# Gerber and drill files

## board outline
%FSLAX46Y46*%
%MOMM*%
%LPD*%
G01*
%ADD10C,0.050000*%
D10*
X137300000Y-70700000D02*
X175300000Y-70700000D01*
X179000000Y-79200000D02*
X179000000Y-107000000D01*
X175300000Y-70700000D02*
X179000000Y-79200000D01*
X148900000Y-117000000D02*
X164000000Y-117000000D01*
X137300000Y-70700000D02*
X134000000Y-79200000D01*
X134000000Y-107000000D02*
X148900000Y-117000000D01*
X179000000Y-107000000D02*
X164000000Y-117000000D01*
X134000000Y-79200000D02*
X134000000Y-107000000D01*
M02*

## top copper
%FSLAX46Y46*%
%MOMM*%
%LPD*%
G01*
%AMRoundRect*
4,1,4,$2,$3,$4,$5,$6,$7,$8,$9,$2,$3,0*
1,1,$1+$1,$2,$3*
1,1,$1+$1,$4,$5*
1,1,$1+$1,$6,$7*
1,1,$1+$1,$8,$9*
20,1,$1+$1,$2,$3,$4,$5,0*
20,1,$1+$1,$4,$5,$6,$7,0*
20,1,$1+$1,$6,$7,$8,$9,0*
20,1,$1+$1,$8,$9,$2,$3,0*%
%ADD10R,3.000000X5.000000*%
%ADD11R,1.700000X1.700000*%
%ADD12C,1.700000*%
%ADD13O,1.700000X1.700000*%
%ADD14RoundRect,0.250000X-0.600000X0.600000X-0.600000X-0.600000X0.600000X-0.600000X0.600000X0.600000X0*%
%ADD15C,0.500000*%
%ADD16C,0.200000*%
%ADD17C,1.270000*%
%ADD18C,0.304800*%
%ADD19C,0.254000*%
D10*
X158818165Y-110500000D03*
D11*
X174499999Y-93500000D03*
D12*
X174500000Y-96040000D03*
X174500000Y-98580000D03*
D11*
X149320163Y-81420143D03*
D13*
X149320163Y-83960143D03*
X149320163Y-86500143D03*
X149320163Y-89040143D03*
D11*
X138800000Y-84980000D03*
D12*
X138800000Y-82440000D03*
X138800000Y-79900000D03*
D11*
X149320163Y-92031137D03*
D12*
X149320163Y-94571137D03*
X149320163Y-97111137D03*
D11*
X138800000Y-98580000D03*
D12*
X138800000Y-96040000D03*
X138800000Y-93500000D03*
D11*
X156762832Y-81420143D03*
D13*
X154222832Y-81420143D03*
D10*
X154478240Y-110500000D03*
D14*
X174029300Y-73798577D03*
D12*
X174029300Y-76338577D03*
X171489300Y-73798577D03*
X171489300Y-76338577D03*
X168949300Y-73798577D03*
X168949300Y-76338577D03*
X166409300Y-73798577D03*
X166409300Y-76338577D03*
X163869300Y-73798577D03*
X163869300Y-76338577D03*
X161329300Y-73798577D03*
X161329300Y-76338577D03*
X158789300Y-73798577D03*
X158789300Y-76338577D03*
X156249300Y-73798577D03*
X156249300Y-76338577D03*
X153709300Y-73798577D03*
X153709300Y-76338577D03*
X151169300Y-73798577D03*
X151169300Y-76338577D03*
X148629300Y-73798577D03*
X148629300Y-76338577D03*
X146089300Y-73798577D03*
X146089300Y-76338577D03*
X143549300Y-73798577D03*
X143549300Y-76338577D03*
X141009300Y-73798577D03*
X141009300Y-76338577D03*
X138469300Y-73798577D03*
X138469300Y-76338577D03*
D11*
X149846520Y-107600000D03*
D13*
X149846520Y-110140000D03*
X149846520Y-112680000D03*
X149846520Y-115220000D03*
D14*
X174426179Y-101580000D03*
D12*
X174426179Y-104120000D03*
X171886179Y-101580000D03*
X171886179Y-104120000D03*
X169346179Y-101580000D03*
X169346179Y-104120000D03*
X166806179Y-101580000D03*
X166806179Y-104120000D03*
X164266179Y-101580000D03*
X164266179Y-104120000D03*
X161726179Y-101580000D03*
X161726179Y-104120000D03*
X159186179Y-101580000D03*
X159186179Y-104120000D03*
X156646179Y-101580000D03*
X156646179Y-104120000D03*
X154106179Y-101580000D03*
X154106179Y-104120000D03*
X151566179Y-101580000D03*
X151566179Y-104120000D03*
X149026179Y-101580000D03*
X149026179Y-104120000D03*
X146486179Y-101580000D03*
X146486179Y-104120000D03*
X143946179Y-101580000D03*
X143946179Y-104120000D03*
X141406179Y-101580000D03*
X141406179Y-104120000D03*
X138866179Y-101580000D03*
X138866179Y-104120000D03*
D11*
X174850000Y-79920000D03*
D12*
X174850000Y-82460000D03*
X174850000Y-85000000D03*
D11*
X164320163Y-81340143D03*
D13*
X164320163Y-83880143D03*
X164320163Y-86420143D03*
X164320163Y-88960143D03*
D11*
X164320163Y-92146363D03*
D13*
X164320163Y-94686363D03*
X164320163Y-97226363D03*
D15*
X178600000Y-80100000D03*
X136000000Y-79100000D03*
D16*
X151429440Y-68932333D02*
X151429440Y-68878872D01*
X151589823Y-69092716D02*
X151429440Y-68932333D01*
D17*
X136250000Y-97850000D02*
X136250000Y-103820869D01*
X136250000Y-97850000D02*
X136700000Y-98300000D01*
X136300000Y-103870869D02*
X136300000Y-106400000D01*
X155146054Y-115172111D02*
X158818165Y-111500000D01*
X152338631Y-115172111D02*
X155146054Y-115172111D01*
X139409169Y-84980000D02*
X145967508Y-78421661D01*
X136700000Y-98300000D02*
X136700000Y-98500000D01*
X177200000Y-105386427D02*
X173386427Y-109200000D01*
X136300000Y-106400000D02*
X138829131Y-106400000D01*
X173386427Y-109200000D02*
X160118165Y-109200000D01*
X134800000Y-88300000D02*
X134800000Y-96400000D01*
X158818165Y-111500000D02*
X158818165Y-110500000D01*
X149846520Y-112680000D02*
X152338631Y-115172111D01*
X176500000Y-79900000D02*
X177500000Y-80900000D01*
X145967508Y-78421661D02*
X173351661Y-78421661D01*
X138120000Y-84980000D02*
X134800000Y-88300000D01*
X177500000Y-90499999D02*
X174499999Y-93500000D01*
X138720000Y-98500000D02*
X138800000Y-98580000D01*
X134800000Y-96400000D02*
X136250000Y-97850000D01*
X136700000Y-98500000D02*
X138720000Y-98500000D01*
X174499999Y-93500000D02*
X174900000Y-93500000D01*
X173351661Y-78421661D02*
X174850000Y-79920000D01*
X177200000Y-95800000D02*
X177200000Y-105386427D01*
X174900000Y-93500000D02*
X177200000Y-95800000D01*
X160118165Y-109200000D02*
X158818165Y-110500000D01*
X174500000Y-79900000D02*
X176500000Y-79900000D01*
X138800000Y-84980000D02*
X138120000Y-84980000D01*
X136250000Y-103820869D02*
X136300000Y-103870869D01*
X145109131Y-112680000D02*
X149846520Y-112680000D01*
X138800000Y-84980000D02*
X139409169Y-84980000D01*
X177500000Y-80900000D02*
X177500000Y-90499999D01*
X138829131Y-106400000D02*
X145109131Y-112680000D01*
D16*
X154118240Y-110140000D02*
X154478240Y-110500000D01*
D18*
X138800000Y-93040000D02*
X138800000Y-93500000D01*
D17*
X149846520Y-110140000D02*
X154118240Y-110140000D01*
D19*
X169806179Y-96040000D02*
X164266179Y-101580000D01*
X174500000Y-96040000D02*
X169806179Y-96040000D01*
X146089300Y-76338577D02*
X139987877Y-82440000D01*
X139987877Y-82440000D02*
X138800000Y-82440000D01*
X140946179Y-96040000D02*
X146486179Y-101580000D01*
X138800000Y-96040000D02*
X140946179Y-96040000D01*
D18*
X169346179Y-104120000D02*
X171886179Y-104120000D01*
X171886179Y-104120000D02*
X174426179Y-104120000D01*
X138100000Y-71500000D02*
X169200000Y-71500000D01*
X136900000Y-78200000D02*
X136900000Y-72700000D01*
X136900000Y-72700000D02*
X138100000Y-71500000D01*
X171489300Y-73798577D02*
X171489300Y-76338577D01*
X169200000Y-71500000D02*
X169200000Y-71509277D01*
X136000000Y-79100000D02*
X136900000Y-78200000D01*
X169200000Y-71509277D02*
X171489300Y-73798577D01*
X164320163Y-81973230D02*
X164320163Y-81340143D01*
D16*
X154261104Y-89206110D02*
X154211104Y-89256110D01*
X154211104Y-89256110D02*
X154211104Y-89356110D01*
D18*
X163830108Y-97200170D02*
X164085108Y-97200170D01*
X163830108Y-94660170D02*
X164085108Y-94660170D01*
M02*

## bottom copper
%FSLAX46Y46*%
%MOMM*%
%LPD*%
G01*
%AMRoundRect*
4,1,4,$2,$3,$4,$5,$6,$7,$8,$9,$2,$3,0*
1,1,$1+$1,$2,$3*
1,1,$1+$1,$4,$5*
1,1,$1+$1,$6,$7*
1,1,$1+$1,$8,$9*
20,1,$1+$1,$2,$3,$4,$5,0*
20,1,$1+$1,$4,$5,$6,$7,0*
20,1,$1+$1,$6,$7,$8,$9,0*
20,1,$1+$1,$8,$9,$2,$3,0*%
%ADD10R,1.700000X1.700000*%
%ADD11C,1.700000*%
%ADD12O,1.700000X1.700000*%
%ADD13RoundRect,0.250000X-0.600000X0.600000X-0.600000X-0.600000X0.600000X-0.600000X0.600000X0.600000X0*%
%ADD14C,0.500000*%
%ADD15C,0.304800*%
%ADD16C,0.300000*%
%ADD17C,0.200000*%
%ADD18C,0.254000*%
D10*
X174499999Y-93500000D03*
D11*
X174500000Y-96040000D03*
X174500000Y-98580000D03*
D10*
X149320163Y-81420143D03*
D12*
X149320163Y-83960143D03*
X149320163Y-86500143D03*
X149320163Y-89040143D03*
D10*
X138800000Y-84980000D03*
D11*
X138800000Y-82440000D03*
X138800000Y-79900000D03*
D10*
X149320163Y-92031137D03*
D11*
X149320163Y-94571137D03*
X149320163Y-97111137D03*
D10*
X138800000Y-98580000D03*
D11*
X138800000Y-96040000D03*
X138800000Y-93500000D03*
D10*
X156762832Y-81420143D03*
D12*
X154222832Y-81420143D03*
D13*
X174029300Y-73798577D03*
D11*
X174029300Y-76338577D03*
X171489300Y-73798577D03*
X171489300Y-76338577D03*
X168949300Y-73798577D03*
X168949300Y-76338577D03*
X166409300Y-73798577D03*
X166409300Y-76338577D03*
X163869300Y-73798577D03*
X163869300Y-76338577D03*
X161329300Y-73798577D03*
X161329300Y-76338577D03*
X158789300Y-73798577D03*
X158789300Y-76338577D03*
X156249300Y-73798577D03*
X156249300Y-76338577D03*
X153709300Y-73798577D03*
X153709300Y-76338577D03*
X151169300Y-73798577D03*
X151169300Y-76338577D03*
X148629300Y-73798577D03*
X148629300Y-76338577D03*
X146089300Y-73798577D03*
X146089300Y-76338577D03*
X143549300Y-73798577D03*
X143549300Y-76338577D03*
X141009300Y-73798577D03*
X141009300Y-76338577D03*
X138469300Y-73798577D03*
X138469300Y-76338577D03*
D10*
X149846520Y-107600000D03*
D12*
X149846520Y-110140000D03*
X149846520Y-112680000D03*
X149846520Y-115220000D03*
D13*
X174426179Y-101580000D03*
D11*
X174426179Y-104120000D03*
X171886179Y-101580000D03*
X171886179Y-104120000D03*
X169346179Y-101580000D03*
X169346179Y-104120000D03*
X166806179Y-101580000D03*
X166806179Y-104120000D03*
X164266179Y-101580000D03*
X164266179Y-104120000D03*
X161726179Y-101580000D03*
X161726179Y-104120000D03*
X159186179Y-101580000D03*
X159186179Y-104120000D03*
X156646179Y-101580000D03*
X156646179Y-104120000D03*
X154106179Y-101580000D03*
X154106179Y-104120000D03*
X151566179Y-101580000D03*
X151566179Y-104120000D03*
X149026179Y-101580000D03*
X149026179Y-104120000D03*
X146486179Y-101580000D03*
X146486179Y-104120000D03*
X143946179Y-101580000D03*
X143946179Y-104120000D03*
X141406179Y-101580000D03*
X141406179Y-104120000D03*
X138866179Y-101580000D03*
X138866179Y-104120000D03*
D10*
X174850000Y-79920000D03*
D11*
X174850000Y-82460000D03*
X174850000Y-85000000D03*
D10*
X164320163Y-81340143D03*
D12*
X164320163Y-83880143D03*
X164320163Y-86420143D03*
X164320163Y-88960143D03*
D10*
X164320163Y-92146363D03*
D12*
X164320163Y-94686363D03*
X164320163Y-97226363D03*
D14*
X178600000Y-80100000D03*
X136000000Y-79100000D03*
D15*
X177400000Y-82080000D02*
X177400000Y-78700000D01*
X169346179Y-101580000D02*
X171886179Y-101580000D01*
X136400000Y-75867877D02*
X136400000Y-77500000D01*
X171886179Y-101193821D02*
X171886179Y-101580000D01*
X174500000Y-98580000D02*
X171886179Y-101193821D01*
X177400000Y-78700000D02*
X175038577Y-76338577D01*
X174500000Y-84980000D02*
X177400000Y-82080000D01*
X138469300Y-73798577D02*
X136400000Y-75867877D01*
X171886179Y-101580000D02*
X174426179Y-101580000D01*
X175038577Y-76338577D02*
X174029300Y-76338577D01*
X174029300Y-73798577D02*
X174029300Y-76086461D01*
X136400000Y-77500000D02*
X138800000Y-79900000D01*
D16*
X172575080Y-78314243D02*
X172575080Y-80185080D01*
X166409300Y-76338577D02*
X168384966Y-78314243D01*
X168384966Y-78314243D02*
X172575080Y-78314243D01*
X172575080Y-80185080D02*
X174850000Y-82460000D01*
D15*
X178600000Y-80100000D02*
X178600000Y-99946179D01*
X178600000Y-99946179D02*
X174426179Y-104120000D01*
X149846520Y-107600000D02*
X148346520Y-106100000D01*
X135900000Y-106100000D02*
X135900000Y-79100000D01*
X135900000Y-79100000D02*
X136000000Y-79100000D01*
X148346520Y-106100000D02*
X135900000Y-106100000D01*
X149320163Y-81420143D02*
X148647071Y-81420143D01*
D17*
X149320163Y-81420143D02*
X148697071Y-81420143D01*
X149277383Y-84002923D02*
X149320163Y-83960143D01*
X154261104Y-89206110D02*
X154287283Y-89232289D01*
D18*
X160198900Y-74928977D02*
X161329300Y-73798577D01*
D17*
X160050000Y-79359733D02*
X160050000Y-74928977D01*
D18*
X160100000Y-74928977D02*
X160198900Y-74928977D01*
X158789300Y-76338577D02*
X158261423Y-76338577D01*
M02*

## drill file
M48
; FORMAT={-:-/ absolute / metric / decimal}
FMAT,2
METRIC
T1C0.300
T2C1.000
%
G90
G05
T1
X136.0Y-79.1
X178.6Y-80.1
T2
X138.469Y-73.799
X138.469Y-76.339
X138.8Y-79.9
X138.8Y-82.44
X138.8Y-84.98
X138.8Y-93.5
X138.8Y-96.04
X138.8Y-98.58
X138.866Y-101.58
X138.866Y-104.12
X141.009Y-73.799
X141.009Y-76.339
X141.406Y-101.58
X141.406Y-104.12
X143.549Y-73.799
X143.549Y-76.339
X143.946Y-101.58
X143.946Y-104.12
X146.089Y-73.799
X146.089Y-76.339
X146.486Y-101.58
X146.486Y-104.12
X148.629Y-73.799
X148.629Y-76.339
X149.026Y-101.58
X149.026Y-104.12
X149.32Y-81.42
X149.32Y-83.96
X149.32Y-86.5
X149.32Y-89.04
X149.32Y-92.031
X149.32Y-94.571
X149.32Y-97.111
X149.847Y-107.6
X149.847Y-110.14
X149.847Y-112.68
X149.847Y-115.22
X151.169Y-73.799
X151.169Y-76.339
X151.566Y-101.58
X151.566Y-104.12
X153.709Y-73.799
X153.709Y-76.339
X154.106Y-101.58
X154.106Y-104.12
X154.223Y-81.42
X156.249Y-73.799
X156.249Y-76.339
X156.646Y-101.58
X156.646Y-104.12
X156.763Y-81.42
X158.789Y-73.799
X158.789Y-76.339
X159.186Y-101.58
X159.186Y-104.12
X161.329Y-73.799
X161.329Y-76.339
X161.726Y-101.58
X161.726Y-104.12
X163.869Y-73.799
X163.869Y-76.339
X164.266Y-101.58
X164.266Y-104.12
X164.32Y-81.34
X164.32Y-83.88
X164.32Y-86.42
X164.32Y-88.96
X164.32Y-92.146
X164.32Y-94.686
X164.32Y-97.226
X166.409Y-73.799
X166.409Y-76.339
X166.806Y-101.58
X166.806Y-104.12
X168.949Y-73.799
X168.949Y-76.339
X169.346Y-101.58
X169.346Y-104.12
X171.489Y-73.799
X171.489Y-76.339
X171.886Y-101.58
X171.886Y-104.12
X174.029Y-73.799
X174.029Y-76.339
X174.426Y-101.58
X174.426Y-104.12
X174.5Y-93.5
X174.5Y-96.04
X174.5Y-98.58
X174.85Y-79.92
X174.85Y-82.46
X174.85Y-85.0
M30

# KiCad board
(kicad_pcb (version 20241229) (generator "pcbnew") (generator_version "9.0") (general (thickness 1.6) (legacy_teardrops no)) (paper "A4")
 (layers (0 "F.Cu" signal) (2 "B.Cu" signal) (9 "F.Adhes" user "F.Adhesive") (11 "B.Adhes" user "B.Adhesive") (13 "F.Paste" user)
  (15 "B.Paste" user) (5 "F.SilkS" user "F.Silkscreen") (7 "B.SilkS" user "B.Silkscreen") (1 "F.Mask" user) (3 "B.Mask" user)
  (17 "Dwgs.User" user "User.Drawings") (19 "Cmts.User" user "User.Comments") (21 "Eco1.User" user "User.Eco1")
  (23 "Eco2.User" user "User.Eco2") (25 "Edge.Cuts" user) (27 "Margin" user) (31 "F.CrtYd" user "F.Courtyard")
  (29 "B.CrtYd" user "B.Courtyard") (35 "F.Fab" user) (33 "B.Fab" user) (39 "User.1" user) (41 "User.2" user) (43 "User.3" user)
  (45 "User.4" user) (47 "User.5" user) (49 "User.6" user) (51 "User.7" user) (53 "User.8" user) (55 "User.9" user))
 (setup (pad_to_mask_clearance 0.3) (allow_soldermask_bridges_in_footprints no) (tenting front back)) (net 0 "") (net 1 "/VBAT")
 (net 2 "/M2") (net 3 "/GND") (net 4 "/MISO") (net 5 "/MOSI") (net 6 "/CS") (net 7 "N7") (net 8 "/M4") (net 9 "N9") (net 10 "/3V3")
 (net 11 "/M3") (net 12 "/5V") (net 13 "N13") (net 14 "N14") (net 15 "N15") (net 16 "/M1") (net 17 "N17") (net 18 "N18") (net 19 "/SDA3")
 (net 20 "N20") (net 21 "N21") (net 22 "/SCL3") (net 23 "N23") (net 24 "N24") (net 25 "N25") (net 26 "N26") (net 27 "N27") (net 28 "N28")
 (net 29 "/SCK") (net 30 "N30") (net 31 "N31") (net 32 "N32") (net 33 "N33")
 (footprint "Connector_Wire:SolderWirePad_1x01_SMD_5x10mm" (layer "F.Cu") (at 158.918165 105.046585)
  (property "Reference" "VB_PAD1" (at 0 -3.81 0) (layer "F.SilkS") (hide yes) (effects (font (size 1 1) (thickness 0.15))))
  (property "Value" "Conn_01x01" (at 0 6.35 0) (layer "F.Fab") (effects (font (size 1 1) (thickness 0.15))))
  (pad "1" smd rect (at -0.1 5.453415) (size 3 5) (layers "F.Cu" "F.Mask" "F.Paste") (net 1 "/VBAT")))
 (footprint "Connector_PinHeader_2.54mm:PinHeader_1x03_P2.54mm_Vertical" (layer "F.Cu") (at 170.094208 95.970955 -45)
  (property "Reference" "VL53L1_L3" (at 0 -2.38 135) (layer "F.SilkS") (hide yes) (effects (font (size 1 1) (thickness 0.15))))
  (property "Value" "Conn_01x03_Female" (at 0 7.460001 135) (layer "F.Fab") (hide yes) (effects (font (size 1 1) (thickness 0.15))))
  (pad "1" thru_hole rect (at 1.368136 -4.862594) (size 1.7 1.7) (drill 1) (layers "*.Cu" "*.Mask") (remove_unused_layers no)
   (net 1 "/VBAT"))
  (pad "2" thru_hole circle (at 3.164188 -3.066543 315) (size 1.7 1.7) (drill 1) (layers "*.Cu" "*.Mask") (remove_unused_layers no)
   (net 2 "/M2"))
  (pad "3" thru_hole circle (at 4.960239 -1.270492 315) (size 1.7 1.7) (drill 1) (layers "*.Cu" "*.Mask") (remove_unused_layers no)
   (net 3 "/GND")))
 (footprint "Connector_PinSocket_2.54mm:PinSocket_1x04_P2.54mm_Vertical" (layer "F.Cu") (at 149.320163 81.420143)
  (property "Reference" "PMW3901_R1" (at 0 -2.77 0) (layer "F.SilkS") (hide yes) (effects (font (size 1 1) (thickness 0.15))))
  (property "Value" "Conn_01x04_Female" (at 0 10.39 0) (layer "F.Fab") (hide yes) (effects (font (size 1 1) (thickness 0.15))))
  (pad "1" thru_hole rect (at 0 0) (size 1.7 1.7) (drill 1) (layers "*.Cu" "*.Mask") (remove_unused_layers no) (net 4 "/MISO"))
  (pad "2" thru_hole oval (at 0 2.54) (size 1.7 1.7) (drill 1) (layers "*.Cu" "*.Mask") (remove_unused_layers no) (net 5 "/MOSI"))
  (pad "3" thru_hole oval (at 0 5.08) (size 1.7 1.7) (drill 1) (layers "*.Cu" "*.Mask") (remove_unused_layers no) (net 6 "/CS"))
  (pad "4" thru_hole oval (at 0 7.62) (size 1.7 1.7) (drill 1) (layers "*.Cu" "*.Mask") (remove_unused_layers no) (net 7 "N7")))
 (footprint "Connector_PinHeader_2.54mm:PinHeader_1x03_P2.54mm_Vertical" (layer "F.Cu") (at 138.5 84.8 -45)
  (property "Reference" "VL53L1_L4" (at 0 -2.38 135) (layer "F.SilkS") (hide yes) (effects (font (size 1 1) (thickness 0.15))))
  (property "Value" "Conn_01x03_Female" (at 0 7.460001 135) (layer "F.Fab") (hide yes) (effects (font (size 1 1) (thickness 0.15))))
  (pad "1" thru_hole rect (at 0.339411 -0.084853 270) (size 1.7 1.7) (drill 1) (layers "*.Cu" "*.Mask") (remove_unused_layers no)
   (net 1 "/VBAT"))
  (pad "2" thru_hole circle (at -1.45664 -1.880904 315) (size 1.7 1.7) (drill 1) (layers "*.Cu" "*.Mask") (remove_unused_layers no)
   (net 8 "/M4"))
  (pad "3" thru_hole circle (at -3.252691 -3.676955 315) (size 1.7 1.7) (drill 1) (layers "*.Cu" "*.Mask") (remove_unused_layers no)
   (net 3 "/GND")))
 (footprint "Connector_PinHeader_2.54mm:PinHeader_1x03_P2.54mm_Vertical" (layer "F.Cu") (at 149.320163 92.031137)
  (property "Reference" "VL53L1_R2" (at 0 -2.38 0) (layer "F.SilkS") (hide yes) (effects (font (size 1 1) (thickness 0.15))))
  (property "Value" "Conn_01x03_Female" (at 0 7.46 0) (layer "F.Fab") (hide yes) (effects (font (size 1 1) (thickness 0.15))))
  (pad "1" thru_hole rect (at 0 0) (size 1.7 1.7) (drill 1) (layers "*.Cu" "*.Mask") (remove_unused_layers no) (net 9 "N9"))
  (pad "2" thru_hole circle (at 0 2.54) (size 1.7 1.7) (drill 1) (layers "*.Cu" "*.Mask") (remove_unused_layers no) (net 3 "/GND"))
  (pad "3" thru_hole circle (at 0 5.08) (size 1.7 1.7) (drill 1) (layers "*.Cu" "*.Mask") (remove_unused_layers no) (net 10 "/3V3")))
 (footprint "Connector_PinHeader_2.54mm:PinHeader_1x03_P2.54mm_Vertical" (layer "F.Cu") (at 142.775639 98.946265 -135)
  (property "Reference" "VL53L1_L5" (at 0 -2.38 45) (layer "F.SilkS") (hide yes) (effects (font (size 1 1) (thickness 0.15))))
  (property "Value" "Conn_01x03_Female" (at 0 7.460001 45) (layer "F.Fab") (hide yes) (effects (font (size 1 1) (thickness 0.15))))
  (pad "1" thru_hole rect (at 2.552213 3.07019 270) (size 1.7 1.7) (drill 1) (layers "*.Cu" "*.Mask") (remove_unused_layers no)
   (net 1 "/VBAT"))
  (pad "2" thru_hole circle (at 0.756162 4.866241 225) (size 1.7 1.7) (drill 1) (layers "*.Cu" "*.Mask") (remove_unused_layers no)
   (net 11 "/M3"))
  (pad "3" thru_hole circle (at -1.03989 6.662292 225) (size 1.7 1.7) (drill 1) (layers "*.Cu" "*.Mask") (remove_unused_layers no)
   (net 3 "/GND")))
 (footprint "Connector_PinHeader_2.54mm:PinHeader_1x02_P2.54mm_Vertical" (layer "F.Cu") (at 156.762832 82.347042 -90)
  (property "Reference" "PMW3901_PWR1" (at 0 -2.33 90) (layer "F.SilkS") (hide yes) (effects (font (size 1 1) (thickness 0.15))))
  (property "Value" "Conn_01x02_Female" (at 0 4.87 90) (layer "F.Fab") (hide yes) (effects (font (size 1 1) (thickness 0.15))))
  (pad "1" thru_hole rect (at -0.926899 0 270) (size 1.7 1.7) (drill 1) (layers "*.Cu" "*.Mask") (remove_unused_layers no) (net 3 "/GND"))
  (pad "2" thru_hole oval (at -0.926899 2.54 270) (size 1.7 1.7) (drill 1) (layers "*.Cu" "*.Mask") (remove_unused_layers no)
   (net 10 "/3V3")))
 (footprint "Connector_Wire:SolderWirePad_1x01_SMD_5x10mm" (layer "F.Cu") (at 153.52824 105.111039)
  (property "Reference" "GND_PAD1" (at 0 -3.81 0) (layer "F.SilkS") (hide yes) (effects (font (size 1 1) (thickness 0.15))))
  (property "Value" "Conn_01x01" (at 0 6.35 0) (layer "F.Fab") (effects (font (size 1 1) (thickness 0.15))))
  (pad "1" smd rect (at 0.95 5.388961) (size 3 5) (layers "F.Cu" "F.Mask" "F.Paste") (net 3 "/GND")))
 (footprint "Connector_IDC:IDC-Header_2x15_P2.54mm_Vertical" (layer "F.Cu") (at 174.0293 73.798577 -90)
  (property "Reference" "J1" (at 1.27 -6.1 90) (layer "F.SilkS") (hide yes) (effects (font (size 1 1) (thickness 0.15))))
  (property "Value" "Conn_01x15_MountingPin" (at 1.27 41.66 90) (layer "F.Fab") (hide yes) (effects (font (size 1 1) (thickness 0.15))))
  (pad "1" thru_hole roundrect (at 0 0 270) (size 1.7 1.7) (drill 1) (layers "*.Cu" "*.Mask") (remove_unused_layers no)
   (roundrect_rratio 0.147059) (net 3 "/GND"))
  (pad "2" thru_hole circle (at 2.54 0 270) (size 1.7 1.7) (drill 1) (layers "*.Cu" "*.Mask") (remove_unused_layers no) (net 3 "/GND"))
  (pad "3" thru_hole circle (at 0 2.54 270) (size 1.7 1.7) (drill 1) (layers "*.Cu" "*.Mask") (remove_unused_layers no) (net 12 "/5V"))
  (pad "4" thru_hole circle (at 2.54 2.54 270) (size 1.7 1.7) (drill 1) (layers "*.Cu" "*.Mask") (remove_unused_layers no) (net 12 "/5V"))
  (pad "5" thru_hole circle (at 0 5.08 270) (size 1.7 1.7) (drill 1) (layers "*.Cu" "*.Mask") (remove_unused_layers no) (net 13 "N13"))
  (pad "6" thru_hole circle (at 2.54 5.08 270) (size 1.7 1.7) (drill 1) (layers "*.Cu" "*.Mask") (remove_unused_layers no) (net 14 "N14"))
  (pad "7" thru_hole circle (at 0 7.62 270) (size 1.7 1.7) (drill 1) (layers "*.Cu" "*.Mask") (remove_unused_layers no) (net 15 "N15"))
  (pad "8" thru_hole circle (at 2.54 7.62 270) (size 1.7 1.7) (drill 1) (layers "*.Cu" "*.Mask") (remove_unused_layers no) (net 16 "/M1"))
  (pad "9" thru_hole circle (at 0 10.16 270) (size 1.7 1.7) (drill 1) (layers "*.Cu" "*.Mask") (remove_unused_layers no) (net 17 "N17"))
  (pad "10" thru_hole circle (at 2.54 10.16 270) (size 1.7 1.7) (drill 1) (layers "*.Cu" "*.Mask") (remove_unused_layers no) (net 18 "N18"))
  (pad "11" thru_hole circle (at 0 12.7 270) (size 1.7 1.7) (drill 1) (layers "*.Cu" "*.Mask") (remove_unused_layers no) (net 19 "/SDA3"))
  (pad "12" thru_hole circle (at 2.54 12.7 270) (size 1.7 1.7) (drill 1) (layers "*.Cu" "*.Mask") (remove_unused_layers no) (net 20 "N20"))
  (pad "13" thru_hole circle (at 0 15.24 270) (size 1.7 1.7) (drill 1) (layers "*.Cu" "*.Mask") (remove_unused_layers no) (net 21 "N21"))
  (pad "14" thru_hole circle (at 2.54 15.24 270) (size 1.7 1.7) (drill 1) (layers "*.Cu" "*.Mask") (remove_unused_layers no)
   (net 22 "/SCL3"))
  (pad "15" thru_hole circle (at 0 17.78 270) (size 1.7 1.7) (drill 1) (layers "*.Cu" "*.Mask") (remove_unused_layers no) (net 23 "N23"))
  (pad "16" thru_hole circle (at 2.54 17.78 270) (size 1.7 1.7) (drill 1) (layers "*.Cu" "*.Mask") (remove_unused_layers no))
  (pad "17" thru_hole circle (at 0 20.32 270) (size 1.7 1.7) (drill 1) (layers "*.Cu" "*.Mask") (remove_unused_layers no))
  (pad "18" thru_hole circle (at 2.54 20.32 270) (size 1.7 1.7) (drill 1) (layers "*.Cu" "*.Mask") (remove_unused_layers no))
  (pad "19" thru_hole circle (at 0 22.86 270) (size 1.7 1.7) (drill 1) (layers "*.Cu" "*.Mask") (remove_unused_layers no))
  (pad "20" thru_hole circle (at 2.54 22.86 270) (size 1.7 1.7) (drill 1) (layers "*.Cu" "*.Mask") (remove_unused_layers no))
  (pad "21" thru_hole circle (at 0 25.4 270) (size 1.7 1.7) (drill 1) (layers "*.Cu" "*.Mask") (remove_unused_layers no))
  (pad "22" thru_hole circle (at 2.54 25.4 270) (size 1.7 1.7) (drill 1) (layers "*.Cu" "*.Mask") (remove_unused_layers no))
  (pad "23" thru_hole circle (at 0 27.94 270) (size 1.7 1.7) (drill 1) (layers "*.Cu" "*.Mask") (remove_unused_layers no))
  (pad "24" thru_hole circle (at 2.54 27.94 270) (size 1.7 1.7) (drill 1) (layers "*.Cu" "*.Mask") (remove_unused_layers no) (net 8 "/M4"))
  (pad "25" thru_hole circle (at 0 30.48 270) (size 1.7 1.7) (drill 1) (layers "*.Cu" "*.Mask") (remove_unused_layers no))
  (pad "26" thru_hole circle (at 2.54 30.48 270) (size 1.7 1.7) (drill 1) (layers "*.Cu" "*.Mask") (remove_unused_layers no))
  (pad "27" thru_hole circle (at 0 33.02 270) (size 1.7 1.7) (drill 1) (layers "*.Cu" "*.Mask") (remove_unused_layers no))
  (pad "28" thru_hole circle (at 2.54 33.02 270) (size 1.7 1.7) (drill 1) (layers "*.Cu" "*.Mask") (remove_unused_layers no))
  (pad "29" thru_hole circle (at 0 35.56 270) (size 1.7 1.7) (drill 1) (layers "*.Cu" "*.Mask") (remove_unused_layers no) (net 3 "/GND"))
  (pad "30" thru_hole circle (at 2.54 35.56 270) (size 1.7 1.7) (drill 1) (layers "*.Cu" "*.Mask") (remove_unused_layers no)))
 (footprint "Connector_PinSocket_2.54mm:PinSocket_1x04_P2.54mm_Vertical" (layer "F.Cu") (at 149.84652 107.6)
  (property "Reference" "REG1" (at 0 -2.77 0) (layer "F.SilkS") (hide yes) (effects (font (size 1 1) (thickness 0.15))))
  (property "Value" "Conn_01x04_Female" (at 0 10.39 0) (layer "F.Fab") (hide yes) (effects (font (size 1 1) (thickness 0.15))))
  (pad "1" thru_hole rect (at 0 0) (size 1.7 1.7) (drill 1) (layers "*.Cu" "*.Mask") (remove_unused_layers no) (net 12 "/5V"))
  (pad "2" thru_hole oval (at 0 2.54) (size 1.7 1.7) (drill 1) (layers "*.Cu" "*.Mask") (remove_unused_layers no) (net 3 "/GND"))
  (pad "3" thru_hole oval (at 0 5.08) (size 1.7 1.7) (drill 1) (layers "*.Cu" "*.Mask") (remove_unused_layers no) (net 1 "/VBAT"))
  (pad "4" thru_hole oval (at 0 7.62) (size 1.7 1.7) (drill 1) (layers "*.Cu" "*.Mask") (remove_unused_layers no) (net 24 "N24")))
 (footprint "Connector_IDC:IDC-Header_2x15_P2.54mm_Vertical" (layer "F.Cu") (at 174.426179 101.58 -90)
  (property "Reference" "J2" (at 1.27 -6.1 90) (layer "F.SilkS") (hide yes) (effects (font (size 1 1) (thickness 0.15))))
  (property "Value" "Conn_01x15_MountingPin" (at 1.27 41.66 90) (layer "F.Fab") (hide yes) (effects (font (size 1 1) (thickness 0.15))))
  (pad "1" thru_hole roundrect (at 0 0 270) (size 1.7 1.7) (drill 1) (layers "*.Cu" "*.Mask") (remove_unused_layers no)
   (roundrect_rratio 0.147059) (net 3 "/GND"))
  (pad "2" thru_hole circle (at 2.54 0 270) (size 1.7 1.7) (drill 1) (layers "*.Cu" "*.Mask") (remove_unused_layers no) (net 10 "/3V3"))
  (pad "3" thru_hole circle (at 0 2.54 270) (size 1.7 1.7) (drill 1) (layers "*.Cu" "*.Mask") (remove_unused_layers no) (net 3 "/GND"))
  (pad "4" thru_hole circle (at 2.54 2.54 270) (size 1.7 1.7) (drill 1) (layers "*.Cu" "*.Mask") (remove_unused_layers no) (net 10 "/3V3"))
  (pad "5" thru_hole circle (at 0 5.08 270) (size 1.7 1.7) (drill 1) (layers "*.Cu" "*.Mask") (remove_unused_layers no) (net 3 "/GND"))
  (pad "6" thru_hole circle (at 2.54 5.08 270) (size 1.7 1.7) (drill 1) (layers "*.Cu" "*.Mask") (remove_unused_layers no) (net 10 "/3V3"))
  (pad "7" thru_hole circle (at 0 7.62 270) (size 1.7 1.7) (drill 1) (layers "*.Cu" "*.Mask") (remove_unused_layers no) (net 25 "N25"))
  (pad "8" thru_hole circle (at 2.54 7.62 270) (size 1.7 1.7) (drill 1) (layers "*.Cu" "*.Mask") (remove_unused_layers no) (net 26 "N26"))
  (pad "9" thru_hole circle (at 0 10.16 270) (size 1.7 1.7) (drill 1) (layers "*.Cu" "*.Mask") (remove_unused_layers no) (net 2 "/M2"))
  (pad "10" thru_hole circle (at 2.54 10.16 270) (size 1.7 1.7) (drill 1) (layers "*.Cu" "*.Mask") (remove_unused_layers no) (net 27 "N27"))
  (pad "11" thru_hole circle (at 0 12.7 270) (size 1.7 1.7) (drill 1) (layers "*.Cu" "*.Mask") (remove_unused_layers no) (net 6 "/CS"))
  (pad "12" thru_hole circle (at 2.54 12.7 270) (size 1.7 1.7) (drill 1) (layers "*.Cu" "*.Mask") (remove_unused_layers no) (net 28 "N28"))
  (pad "13" thru_hole circle (at 0 15.24 270) (size 1.7 1.7) (drill 1) (layers "*.Cu" "*.Mask") (remove_unused_layers no) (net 5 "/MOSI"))
  (pad "14" thru_hole circle (at 2.54 15.24 270) (size 1.7 1.7) (drill 1) (layers "*.Cu" "*.Mask") (remove_unused_layers no))
  (pad "15" thru_hole circle (at 0 17.78 270) (size 1.7 1.7) (drill 1) (layers "*.Cu" "*.Mask") (remove_unused_layers no) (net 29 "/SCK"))
  (pad "16" thru_hole circle (at 2.54 17.78 270) (size 1.7 1.7) (drill 1) (layers "*.Cu" "*.Mask") (remove_unused_layers no) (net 4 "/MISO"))
  (pad "17" thru_hole circle (at 0 20.32 270) (size 1.7 1.7) (drill 1) (layers "*.Cu" "*.Mask") (remove_unused_layers no))
  (pad "18" thru_hole circle (at 2.54 20.32 270) (size 1.7 1.7) (drill 1) (layers "*.Cu" "*.Mask") (remove_unused_layers no))
  (pad "19" thru_hole circle (at 0 22.86 270) (size 1.7 1.7) (drill 1) (layers "*.Cu" "*.Mask") (remove_unused_layers no))
  (pad "20" thru_hole circle (at 2.54 22.86 270) (size 1.7 1.7) (drill 1) (layers "*.Cu" "*.Mask") (remove_unused_layers no))
  (pad "21" thru_hole circle (at 0 25.4 270) (size 1.7 1.7) (drill 1) (layers "*.Cu" "*.Mask") (remove_unused_layers no))
  (pad "22" thru_hole circle (at 2.54 25.4 270) (size 1.7 1.7) (drill 1) (layers "*.Cu" "*.Mask") (remove_unused_layers no))
  (pad "23" thru_hole circle (at 0 27.94 270) (size 1.7 1.7) (drill 1) (layers "*.Cu" "*.Mask") (remove_unused_layers no) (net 11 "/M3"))
  (pad "24" thru_hole circle (at 2.54 27.94 270) (size 1.7 1.7) (drill 1) (layers "*.Cu" "*.Mask") (remove_unused_layers no))
  (pad "25" thru_hole circle (at 0 30.48 270) (size 1.7 1.7) (drill 1) (layers "*.Cu" "*.Mask") (remove_unused_layers no))
  (pad "26" thru_hole circle (at 2.54 30.48 270) (size 1.7 1.7) (drill 1) (layers "*.Cu" "*.Mask") (remove_unused_layers no))
  (pad "27" thru_hole circle (at 0 33.02 270) (size 1.7 1.7) (drill 1) (layers "*.Cu" "*.Mask") (remove_unused_layers no))
  (pad "28" thru_hole circle (at 2.54 33.02 270) (size 1.7 1.7) (drill 1) (layers "*.Cu" "*.Mask") (remove_unused_layers no))
  (pad "29" thru_hole circle (at 0 35.56 270) (size 1.7 1.7) (drill 1) (layers "*.Cu" "*.Mask") (remove_unused_layers no) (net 3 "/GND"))
  (pad "30" thru_hole circle (at 2.54 35.56 270) (size 1.7 1.7) (drill 1) (layers "*.Cu" "*.Mask") (remove_unused_layers no)))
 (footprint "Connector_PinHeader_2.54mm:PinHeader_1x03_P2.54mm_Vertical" (layer "F.Cu") (at 174.85 79.92)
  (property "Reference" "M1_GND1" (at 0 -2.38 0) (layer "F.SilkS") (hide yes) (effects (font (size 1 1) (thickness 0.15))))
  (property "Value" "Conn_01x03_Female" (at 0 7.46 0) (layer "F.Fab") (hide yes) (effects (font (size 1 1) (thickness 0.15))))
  (pad "1" thru_hole rect (at 0 0) (size 1.7 1.7) (drill 1) (layers "*.Cu" "*.Mask") (remove_unused_layers no) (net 1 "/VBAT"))
  (pad "2" thru_hole circle (at 0 2.54) (size 1.7 1.7) (drill 1) (layers "*.Cu" "*.Mask") (remove_unused_layers no) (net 16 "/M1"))
  (pad "3" thru_hole circle (at 0 5.08) (size 1.7 1.7) (drill 1) (layers "*.Cu" "*.Mask") (remove_unused_layers no) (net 3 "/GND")))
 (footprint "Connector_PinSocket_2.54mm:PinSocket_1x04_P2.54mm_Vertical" (layer "F.Cu") (at 164.320163 81.340143)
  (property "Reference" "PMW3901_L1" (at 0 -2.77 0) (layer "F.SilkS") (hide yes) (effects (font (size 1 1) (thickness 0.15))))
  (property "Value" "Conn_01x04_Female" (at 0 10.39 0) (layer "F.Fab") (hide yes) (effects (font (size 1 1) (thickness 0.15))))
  (pad "1" thru_hole rect (at 0 0) (size 1.7 1.7) (drill 1) (layers "*.Cu" "*.Mask") (remove_unused_layers no) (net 29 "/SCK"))
  (pad "2" thru_hole oval (at 0 2.54) (size 1.7 1.7) (drill 1) (layers "*.Cu" "*.Mask") (remove_unused_layers no) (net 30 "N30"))
  (pad "3" thru_hole oval (at 0 5.08) (size 1.7 1.7) (drill 1) (layers "*.Cu" "*.Mask") (remove_unused_layers no) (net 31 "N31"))
  (pad "4" thru_hole oval (at 0 7.62) (size 1.7 1.7) (drill 1) (layers "*.Cu" "*.Mask") (remove_unused_layers no) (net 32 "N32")))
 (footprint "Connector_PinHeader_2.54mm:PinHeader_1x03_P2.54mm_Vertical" (layer "F.Cu") (at 164.320163 92.146363)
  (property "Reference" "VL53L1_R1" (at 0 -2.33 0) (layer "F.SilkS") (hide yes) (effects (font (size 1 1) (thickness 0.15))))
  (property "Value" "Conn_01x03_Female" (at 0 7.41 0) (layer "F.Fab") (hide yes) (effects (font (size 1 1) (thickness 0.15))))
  (pad "1" thru_hole rect (at 0 0) (size 1.7 1.7) (drill 1) (layers "*.Cu" "*.Mask") (remove_unused_layers no) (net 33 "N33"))
  (pad "2" thru_hole oval (at 0 2.54) (size 1.7 1.7) (drill 1) (layers "*.Cu" "*.Mask") (remove_unused_layers no) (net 22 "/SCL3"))
  (pad "3" thru_hole oval (at 0 5.08) (size 1.7 1.7) (drill 1) (layers "*.Cu" "*.Mask") (remove_unused_layers no) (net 19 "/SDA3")))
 (gr_line (start 137.3 70.7) (end 175.3 70.7) (stroke (width 0.05) (type solid)) (layer "Edge.Cuts"))
 (gr_line (start 179 79.2) (end 179 107) (stroke (width 0.05) (type solid)) (layer "Edge.Cuts"))
 (gr_line (start 175.3 70.7) (end 179 79.2) (stroke (width 0.05) (type solid)) (layer "Edge.Cuts"))
 (gr_line (start 148.9 117) (end 164 117) (stroke (width 0.05) (type solid)) (layer "Edge.Cuts"))
 (gr_line (start 137.3 70.7) (end 134 79.2) (stroke (width 0.05) (type solid)) (layer "Edge.Cuts"))
 (gr_line (start 134 107) (end 148.9 117) (stroke (width 0.05) (type solid)) (layer "Edge.Cuts"))
 (gr_line (start 179 107) (end 164 117) (stroke (width 0.05) (type solid)) (layer "Edge.Cuts"))
 (gr_line (start 134 79.2) (end 134 107) (stroke (width 0.05) (type solid)) (layer "Edge.Cuts"))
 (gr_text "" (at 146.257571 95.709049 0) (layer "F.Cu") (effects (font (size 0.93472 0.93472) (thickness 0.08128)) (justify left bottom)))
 (segment (start 151.42944 68.932333) (end 151.42944 68.878872) (width 0.2) (layer "F.Cu") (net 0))
 (segment (start 151.589823 69.092716) (end 151.42944 68.932333) (width 0.2) (layer "F.Cu") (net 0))
 (segment (start 136.25 97.85) (end 136.25 103.820869) (width 1.27) (layer "F.Cu") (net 1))
 (segment (start 136.25 97.85) (end 136.7 98.3) (width 1.27) (layer "F.Cu") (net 1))
 (segment (start 136.3 103.870869) (end 136.3 106.4) (width 1.27) (layer "F.Cu") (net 1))
 (segment (start 155.146054 115.172111) (end 158.818165 111.5) (width 1.27) (layer "F.Cu") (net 1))
 (segment (start 152.338631 115.172111) (end 155.146054 115.172111) (width 1.27) (layer "F.Cu") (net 1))
 (segment (start 139.409169 84.98) (end 145.967508 78.421661) (width 1.27) (layer "F.Cu") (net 1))
 (segment (start 136.7 98.3) (end 136.7 98.5) (width 1.27) (layer "F.Cu") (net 1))
 (segment (start 177.2 105.386427) (end 173.386427 109.2) (width 1.27) (layer "F.Cu") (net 1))
 (segment (start 136.3 106.4) (end 138.829131 106.4) (width 1.27) (layer "F.Cu") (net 1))
 (segment (start 173.386427 109.2) (end 160.118165 109.2) (width 1.27) (layer "F.Cu") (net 1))
 (segment (start 134.8 88.3) (end 134.8 96.4) (width 1.27) (layer "F.Cu") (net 1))
 (segment (start 158.818165 111.5) (end 158.818165 110.5) (width 1.27) (layer "F.Cu") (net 1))
 (segment (start 149.84652 112.68) (end 152.338631 115.172111) (width 1.27) (layer "F.Cu") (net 1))
 (segment (start 176.5 79.9) (end 177.5 80.9) (width 1.27) (layer "F.Cu") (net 1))
 (segment (start 145.967508 78.421661) (end 173.351661 78.421661) (width 1.27) (layer "F.Cu") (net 1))
 (segment (start 138.12 84.98) (end 134.8 88.3) (width 1.27) (layer "F.Cu") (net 1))
 (segment (start 177.5 90.499999) (end 174.499999 93.5) (width 1.27) (layer "F.Cu") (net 1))
 (segment (start 138.72 98.5) (end 138.8 98.58) (width 1.27) (layer "F.Cu") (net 1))
 (segment (start 134.8 96.4) (end 136.25 97.85) (width 1.27) (layer "F.Cu") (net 1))
 (segment (start 136.7 98.5) (end 138.72 98.5) (width 1.27) (layer "F.Cu") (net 1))
 (segment (start 174.499999 93.5) (end 174.9 93.5) (width 1.27) (layer "F.Cu") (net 1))
 (segment (start 173.351661 78.421661) (end 174.85 79.92) (width 1.27) (layer "F.Cu") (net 1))
 (segment (start 177.2 95.8) (end 177.2 105.386427) (width 1.27) (layer "F.Cu") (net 1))
 (segment (start 174.9 93.5) (end 177.2 95.8) (width 1.27) (layer "F.Cu") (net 1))
 (segment (start 160.118165 109.2) (end 158.818165 110.5) (width 1.27) (layer "F.Cu") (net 1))
 (segment (start 174.5 79.9) (end 176.5 79.9) (width 1.27) (layer "F.Cu") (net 1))
 (segment (start 138.8 84.98) (end 138.12 84.98) (width 1.27) (layer "F.Cu") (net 1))
 (segment (start 136.25 103.820869) (end 136.3 103.870869) (width 1.27) (layer "F.Cu") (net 1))
 (segment (start 145.109131 112.68) (end 149.84652 112.68) (width 1.27) (layer "F.Cu") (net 1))
 (segment (start 138.8 84.98) (end 139.409169 84.98) (width 1.27) (layer "F.Cu") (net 1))
 (segment (start 177.5 80.9) (end 177.5 90.499999) (width 1.27) (layer "F.Cu") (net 1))
 (segment (start 138.829131 106.4) (end 145.109131 112.68) (width 1.27) (layer "F.Cu") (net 1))
 (segment (start 154.11824 110.14) (end 154.47824 110.5) (width 0.2) (layer "F.Cu") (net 3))
 (segment (start 138.8 93.04) (end 138.8 93.5) (width 0.3048) (layer "F.Cu") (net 3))
 (segment (start 149.84652 110.14) (end 154.11824 110.14) (width 1.27) (layer "F.Cu") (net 3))
 (segment (start 177.4 82.08) (end 177.4 78.7) (width 0.3048) (layer "B.Cu") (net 3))
 (segment (start 169.346179 101.58) (end 171.886179 101.58) (width 0.3048) (layer "B.Cu") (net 3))
 (segment (start 136.4 75.867877) (end 136.4 77.5) (width 0.3048) (layer "B.Cu") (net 3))
 (segment (start 171.886179 101.193821) (end 171.886179 101.58) (width 0.3048) (layer "B.Cu") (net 3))
 (segment (start 174.5 98.58) (end 171.886179 101.193821) (width 0.3048) (layer "B.Cu") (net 3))
 (segment (start 177.4 78.7) (end 175.038577 76.338577) (width 0.3048) (layer "B.Cu") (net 3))
 (segment (start 174.5 84.98) (end 177.4 82.08) (width 0.3048) (layer "B.Cu") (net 3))
 (segment (start 138.4693 73.798577) (end 136.4 75.867877) (width 0.3048) (layer "B.Cu") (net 3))
 (segment (start 171.886179 101.58) (end 174.426179 101.58) (width 0.3048) (layer "B.Cu") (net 3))
 (segment (start 175.038577 76.338577) (end 174.0293 76.338577) (width 0.3048) (layer "B.Cu") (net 3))
 (segment (start 174.0293 73.798577) (end 174.0293 76.086461) (width 0.3048) (layer "B.Cu") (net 3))
 (segment (start 136.4 77.5) (end 138.8 79.9) (width 0.3048) (layer "B.Cu") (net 3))
 (segment (start 172.57508 78.314243) (end 172.57508 80.18508) (width 0.3) (layer "B.Cu") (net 16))
 (segment (start 166.4093 76.338577) (end 168.384966 78.314243) (width 0.3) (layer "B.Cu") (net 16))
 (segment (start 168.384966 78.314243) (end 172.57508 78.314243) (width 0.3) (layer "B.Cu") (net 16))
 (segment (start 172.57508 80.18508) (end 174.85 82.46) (width 0.3) (layer "B.Cu") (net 16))
 (segment (start 169.806179 96.04) (end 164.266179 101.58) (width 0.254) (layer "F.Cu") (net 2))
 (segment (start 174.5 96.04) (end 169.806179 96.04) (width 0.254) (layer "F.Cu") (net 2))
 (segment (start 146.0893 76.338577) (end 139.987877 82.44) (width 0.254) (layer "F.Cu") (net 8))
 (segment (start 139.987877 82.44) (end 138.8 82.44) (width 0.254) (layer "F.Cu") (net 8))
 (segment (start 140.946179 96.04) (end 146.486179 101.58) (width 0.254) (layer "F.Cu") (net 11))
 (segment (start 138.8 96.04) (end 140.946179 96.04) (width 0.254) (layer "F.Cu") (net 11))
 (segment (start 169.346179 104.12) (end 171.886179 104.12) (width 0.3048) (layer "F.Cu") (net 10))
 (segment (start 171.886179 104.12) (end 174.426179 104.12) (width 0.3048) (layer "F.Cu") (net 10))
 (via (at 178.6 80.1) (size 0.5) (drill 0.3) (layers "F.Cu" "B.Cu") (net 10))
 (segment (start 178.6 80.1) (end 178.6 99.946179) (width 0.3048) (layer "B.Cu") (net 10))
 (segment (start 178.6 99.946179) (end 174.426179 104.12) (width 0.3048) (layer "B.Cu") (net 10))
 (segment (start 138.1 71.5) (end 169.2 71.5) (width 0.3048) (layer "F.Cu") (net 12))
 (segment (start 136.9 78.2) (end 136.9 72.7) (width 0.3048) (layer "F.Cu") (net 12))
 (segment (start 136.9 72.7) (end 138.1 71.5) (width 0.3048) (layer "F.Cu") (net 12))
 (segment (start 171.4893 73.798577) (end 171.4893 76.338577) (width 0.3048) (layer "F.Cu") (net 12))
 (segment (start 169.2 71.5) (end 169.2 71.509277) (width 0.3048) (layer "F.Cu") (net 12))
 (segment (start 136 79.1) (end 136.9 78.2) (width 0.3048) (layer "F.Cu") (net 12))
 (segment (start 169.2 71.509277) (end 171.4893 73.798577) (width 0.3048) (layer "F.Cu") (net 12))
 (via (at 136 79.1) (size 0.5) (drill 0.3) (layers "F.Cu" "B.Cu") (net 12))
 (segment (start 149.84652 107.6) (end 148.34652 106.1) (width 0.3048) (layer "B.Cu") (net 12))
 (segment (start 135.9 106.1) (end 135.9 79.1) (width 0.3048) (layer "B.Cu") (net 12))
 (segment (start 135.9 79.1) (end 136 79.1) (width 0.3048) (layer "B.Cu") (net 12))
 (segment (start 148.34652 106.1) (end 135.9 106.1) (width 0.3048) (layer "B.Cu") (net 12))
 (segment (start 164.320163 81.97323) (end 164.320163 81.340143) (width 0.3048) (layer "F.Cu") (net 29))
 (segment (start 149.320163 81.420143) (end 148.647071 81.420143) (width 0.3048) (layer "B.Cu") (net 4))
 (segment (start 149.320163 81.420143) (end 148.697071 81.420143) (width 0.2) (layer "B.Cu") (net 4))
 (segment (start 149.277383 84.002923) (end 149.320163 83.960143) (width 0.2) (layer "B.Cu") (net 5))
 (segment (start 154.261104 89.20611) (end 154.211104 89.25611) (width 0.2) (layer "F.Cu") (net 6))
 (segment (start 154.211104 89.25611) (end 154.211104 89.35611) (width 0.2) (layer "F.Cu") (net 6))
 (segment (start 154.261104 89.20611) (end 154.287283 89.232289) (width 0.2) (layer "B.Cu") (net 6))
 (segment (start 163.830108 97.20017) (end 164.085108 97.20017) (width 0.3048) (layer "F.Cu") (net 19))
 (segment (start 160.1989 74.928977) (end 161.3293 73.798577) (width 0.254) (layer "B.Cu") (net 19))
 (segment (start 160.05 79.359733) (end 160.05 74.928977) (width 0.2) (layer "B.Cu") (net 19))
 (segment (start 160.1 74.928977) (end 160.1989 74.928977) (width 0.254) (layer "B.Cu") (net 19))
 (segment (start 163.830108 94.66017) (end 164.085108 94.66017) (width 0.3048) (layer "F.Cu") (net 22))
 (segment (start 158.7893 76.338577) (end 158.261423 76.338577) (width 0.254) (layer "B.Cu") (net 22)))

